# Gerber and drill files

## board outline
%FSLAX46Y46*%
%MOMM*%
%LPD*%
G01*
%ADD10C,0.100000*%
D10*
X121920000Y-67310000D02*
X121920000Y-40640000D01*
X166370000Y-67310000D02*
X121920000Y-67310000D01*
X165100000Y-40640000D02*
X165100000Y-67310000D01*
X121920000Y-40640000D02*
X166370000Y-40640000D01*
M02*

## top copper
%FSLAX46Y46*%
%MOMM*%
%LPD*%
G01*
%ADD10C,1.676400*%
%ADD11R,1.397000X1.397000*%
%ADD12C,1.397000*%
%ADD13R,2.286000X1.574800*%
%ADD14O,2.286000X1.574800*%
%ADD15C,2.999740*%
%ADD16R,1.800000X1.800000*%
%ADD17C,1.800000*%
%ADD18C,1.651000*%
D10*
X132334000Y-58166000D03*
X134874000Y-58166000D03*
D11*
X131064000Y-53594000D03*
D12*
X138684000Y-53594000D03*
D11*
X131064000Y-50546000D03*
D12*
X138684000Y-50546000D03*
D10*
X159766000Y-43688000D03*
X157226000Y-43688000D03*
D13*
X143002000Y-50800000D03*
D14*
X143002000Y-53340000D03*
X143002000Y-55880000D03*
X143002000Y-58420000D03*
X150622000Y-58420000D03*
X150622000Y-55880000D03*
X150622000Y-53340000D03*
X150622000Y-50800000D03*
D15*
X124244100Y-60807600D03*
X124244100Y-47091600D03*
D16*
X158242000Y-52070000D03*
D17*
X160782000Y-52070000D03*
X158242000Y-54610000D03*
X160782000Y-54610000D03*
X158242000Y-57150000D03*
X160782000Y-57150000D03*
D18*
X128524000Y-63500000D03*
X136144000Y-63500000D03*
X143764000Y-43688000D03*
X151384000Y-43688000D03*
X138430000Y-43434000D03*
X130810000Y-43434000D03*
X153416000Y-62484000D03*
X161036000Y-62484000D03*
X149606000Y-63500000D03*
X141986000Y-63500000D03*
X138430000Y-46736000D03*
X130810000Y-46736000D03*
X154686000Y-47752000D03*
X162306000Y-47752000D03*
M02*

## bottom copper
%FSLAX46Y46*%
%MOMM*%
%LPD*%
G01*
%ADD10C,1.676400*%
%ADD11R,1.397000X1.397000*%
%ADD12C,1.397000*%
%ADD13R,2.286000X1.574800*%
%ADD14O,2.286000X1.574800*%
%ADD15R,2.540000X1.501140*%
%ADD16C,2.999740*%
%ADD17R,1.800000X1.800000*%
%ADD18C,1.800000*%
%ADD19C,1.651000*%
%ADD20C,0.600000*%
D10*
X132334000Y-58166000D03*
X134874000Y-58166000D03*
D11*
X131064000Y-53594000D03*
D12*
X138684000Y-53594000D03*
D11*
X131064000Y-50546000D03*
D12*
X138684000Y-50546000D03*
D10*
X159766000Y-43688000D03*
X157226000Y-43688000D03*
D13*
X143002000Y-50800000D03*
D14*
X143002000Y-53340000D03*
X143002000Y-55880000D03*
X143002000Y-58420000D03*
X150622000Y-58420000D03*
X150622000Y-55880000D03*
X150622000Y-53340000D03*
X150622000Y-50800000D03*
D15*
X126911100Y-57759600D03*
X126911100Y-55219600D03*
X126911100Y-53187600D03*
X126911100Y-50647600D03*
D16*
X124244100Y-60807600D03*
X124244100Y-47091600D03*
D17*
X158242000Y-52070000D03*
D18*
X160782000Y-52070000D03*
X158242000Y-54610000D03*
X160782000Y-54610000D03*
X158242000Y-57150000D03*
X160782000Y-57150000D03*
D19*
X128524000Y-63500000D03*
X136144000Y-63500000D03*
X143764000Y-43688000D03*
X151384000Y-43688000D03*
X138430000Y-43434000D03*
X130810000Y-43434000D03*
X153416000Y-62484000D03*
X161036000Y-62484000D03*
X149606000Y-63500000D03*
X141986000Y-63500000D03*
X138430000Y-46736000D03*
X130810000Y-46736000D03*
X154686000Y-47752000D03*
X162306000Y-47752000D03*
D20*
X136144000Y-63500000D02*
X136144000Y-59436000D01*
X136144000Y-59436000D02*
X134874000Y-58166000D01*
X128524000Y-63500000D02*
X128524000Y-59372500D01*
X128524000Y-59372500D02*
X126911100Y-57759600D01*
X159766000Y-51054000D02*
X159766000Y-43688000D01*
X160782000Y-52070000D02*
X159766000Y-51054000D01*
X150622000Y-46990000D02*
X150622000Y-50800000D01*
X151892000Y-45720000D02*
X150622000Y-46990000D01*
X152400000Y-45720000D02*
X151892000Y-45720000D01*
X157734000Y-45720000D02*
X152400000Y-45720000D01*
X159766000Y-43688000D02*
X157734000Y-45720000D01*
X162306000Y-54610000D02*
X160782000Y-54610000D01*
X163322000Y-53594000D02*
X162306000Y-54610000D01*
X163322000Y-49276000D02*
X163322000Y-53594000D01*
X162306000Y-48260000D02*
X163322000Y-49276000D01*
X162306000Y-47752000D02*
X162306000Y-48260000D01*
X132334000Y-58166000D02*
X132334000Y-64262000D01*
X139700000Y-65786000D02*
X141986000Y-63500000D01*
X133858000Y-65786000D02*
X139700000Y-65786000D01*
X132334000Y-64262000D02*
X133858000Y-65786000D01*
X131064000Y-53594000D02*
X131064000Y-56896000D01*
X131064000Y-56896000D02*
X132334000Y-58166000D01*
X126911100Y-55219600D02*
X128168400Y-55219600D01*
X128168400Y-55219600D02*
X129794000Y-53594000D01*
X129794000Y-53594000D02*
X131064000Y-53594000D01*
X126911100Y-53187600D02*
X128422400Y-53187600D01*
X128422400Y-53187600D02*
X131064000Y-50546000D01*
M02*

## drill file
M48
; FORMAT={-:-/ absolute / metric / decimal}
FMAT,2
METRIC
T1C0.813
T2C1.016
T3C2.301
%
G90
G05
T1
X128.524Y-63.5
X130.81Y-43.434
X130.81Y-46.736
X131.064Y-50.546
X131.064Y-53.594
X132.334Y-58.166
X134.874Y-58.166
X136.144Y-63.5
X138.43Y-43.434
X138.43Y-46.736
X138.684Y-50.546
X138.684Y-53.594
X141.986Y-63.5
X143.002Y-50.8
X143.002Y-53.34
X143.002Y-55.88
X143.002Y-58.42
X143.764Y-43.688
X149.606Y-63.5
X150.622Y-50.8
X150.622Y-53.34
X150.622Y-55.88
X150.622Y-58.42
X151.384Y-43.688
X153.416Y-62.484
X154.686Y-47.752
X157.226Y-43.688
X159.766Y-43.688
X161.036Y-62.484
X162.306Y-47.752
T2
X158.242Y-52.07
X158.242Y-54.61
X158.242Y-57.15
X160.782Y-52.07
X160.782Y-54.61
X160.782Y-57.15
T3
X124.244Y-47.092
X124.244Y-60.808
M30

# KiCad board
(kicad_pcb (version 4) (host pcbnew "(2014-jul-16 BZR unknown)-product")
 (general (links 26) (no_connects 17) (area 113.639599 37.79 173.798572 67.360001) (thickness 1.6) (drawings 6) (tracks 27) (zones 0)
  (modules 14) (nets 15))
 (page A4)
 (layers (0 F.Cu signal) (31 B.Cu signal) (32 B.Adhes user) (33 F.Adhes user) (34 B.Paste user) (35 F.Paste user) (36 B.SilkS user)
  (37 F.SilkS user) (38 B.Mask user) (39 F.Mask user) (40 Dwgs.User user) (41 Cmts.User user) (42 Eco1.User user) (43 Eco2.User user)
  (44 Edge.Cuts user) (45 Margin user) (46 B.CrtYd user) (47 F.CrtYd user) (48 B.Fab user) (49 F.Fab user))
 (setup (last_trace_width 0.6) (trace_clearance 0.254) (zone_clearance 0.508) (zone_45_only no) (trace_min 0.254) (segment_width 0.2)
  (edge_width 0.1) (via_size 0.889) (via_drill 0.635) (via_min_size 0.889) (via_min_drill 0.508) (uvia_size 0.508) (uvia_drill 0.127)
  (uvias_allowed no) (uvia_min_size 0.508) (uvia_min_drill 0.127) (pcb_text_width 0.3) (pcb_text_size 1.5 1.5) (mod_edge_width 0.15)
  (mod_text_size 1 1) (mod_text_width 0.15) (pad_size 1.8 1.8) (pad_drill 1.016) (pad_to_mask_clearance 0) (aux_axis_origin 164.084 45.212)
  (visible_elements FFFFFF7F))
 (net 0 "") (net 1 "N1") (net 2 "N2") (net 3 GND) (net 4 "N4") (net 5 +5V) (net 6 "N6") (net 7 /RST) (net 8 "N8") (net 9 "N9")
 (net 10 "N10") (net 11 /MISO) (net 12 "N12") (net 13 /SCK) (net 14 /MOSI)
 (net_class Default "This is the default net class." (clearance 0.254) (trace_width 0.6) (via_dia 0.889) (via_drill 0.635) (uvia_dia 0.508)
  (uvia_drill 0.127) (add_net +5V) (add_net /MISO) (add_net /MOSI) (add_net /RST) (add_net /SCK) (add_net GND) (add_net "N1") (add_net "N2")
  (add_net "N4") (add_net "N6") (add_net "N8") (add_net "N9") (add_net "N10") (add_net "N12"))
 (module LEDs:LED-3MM (layer F.Cu) (at 133.604 58.166)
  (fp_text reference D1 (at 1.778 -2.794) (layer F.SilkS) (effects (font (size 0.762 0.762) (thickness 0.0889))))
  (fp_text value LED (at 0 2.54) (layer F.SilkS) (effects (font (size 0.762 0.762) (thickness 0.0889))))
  (pad 1 thru_hole circle (at -1.27 0) (size 1.6764 1.6764) (drill 0.8128) (layers *.Cu *.Mask F.SilkS) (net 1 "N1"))
  (pad 2 thru_hole circle (at 1.27 0) (size 1.6764 1.6764) (drill 0.8128) (layers *.Cu *.Mask F.SilkS) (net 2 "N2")))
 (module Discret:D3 (layer F.Cu) (at 134.874 53.594 180)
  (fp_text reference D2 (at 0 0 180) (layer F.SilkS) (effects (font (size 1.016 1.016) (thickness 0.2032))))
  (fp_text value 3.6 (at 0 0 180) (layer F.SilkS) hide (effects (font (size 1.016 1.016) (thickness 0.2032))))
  (pad 2 thru_hole rect (at 3.81 0 180) (size 1.397 1.397) (drill 0.8128) (layers *.Cu *.Mask F.SilkS) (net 1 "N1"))
  (pad 1 thru_hole circle (at -3.81 0 180) (size 1.397 1.397) (drill 0.8128) (layers *.Cu *.Mask F.SilkS) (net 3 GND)))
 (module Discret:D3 (layer F.Cu) (at 134.874 50.546 180)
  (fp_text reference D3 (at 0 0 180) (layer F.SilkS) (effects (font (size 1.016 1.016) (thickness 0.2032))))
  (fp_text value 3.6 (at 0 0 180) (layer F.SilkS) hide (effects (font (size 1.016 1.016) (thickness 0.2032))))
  (pad 2 thru_hole rect (at 3.81 0 180) (size 1.397 1.397) (drill 0.8128) (layers *.Cu *.Mask F.SilkS) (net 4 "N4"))
  (pad 1 thru_hole circle (at -3.81 0 180) (size 1.397 1.397) (drill 0.8128) (layers *.Cu *.Mask F.SilkS) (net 3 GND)))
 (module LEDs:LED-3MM (layer F.Cu) (at 158.496 43.688 180)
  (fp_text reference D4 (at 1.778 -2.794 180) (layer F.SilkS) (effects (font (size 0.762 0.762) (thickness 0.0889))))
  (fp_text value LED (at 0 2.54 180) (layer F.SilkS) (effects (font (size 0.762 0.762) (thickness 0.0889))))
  (pad 1 thru_hole circle (at -1.27 0 180) (size 1.6764 1.6764) (drill 0.8128) (layers *.Cu *.Mask F.SilkS) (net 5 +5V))
  (pad 2 thru_hole circle (at 1.27 0 180) (size 1.6764 1.6764) (drill 0.8128) (layers *.Cu *.Mask F.SilkS) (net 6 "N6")))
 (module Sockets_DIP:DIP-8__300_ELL (layer F.Cu) (at 146.812 54.61 270)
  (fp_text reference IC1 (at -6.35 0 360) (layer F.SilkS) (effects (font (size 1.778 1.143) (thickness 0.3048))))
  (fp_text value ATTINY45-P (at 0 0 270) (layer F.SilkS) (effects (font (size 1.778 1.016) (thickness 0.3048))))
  (pad 1 thru_hole rect (at -3.81 3.81 270) (size 1.5748 2.286) (drill 0.8128) (layers *.Cu *.Mask F.SilkS) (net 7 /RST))
  (pad 2 thru_hole oval (at -1.27 3.81 270) (size 1.5748 2.286) (drill 0.8128) (layers *.Cu *.Mask F.SilkS) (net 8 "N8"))
  (pad 3 thru_hole oval (at 1.27 3.81 270) (size 1.5748 2.286) (drill 0.8128) (layers *.Cu *.Mask F.SilkS) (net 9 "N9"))
  (pad 4 thru_hole oval (at 3.81 3.81 270) (size 1.5748 2.286) (drill 0.8128) (layers *.Cu *.Mask F.SilkS) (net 3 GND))
  (pad 5 thru_hole oval (at 3.81 -3.81 270) (size 1.5748 2.286) (drill 0.8128) (layers *.Cu *.Mask F.SilkS) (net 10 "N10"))
  (pad 6 thru_hole oval (at 1.27 -3.81 270) (size 1.5748 2.286) (drill 0.8128) (layers *.Cu *.Mask F.SilkS) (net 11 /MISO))
  (pad 7 thru_hole oval (at -1.27 -3.81 270) (size 1.5748 2.286) (drill 0.8128) (layers *.Cu *.Mask F.SilkS) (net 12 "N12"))
  (pad 8 thru_hole oval (at -3.81 -3.81 270) (size 1.5748 2.286) (drill 0.8128) (layers *.Cu *.Mask F.SilkS) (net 5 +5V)))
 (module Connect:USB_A (layer F.Cu) (at 126.9111 54.2036 180)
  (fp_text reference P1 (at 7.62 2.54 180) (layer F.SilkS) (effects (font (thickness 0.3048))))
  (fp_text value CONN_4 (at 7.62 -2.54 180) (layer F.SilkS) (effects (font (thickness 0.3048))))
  (pad 4 smd rect (at 0 -3.556 180) (size 2.54 1.50114) (layers B.Cu F.Paste F.Mask) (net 3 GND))
  (pad 3 smd rect (at 0 -1.016 180) (size 2.54 1.50114) (layers B.Cu F.Paste F.Mask) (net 1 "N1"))
  (pad 2 smd rect (at 0 1.016 180) (size 2.54 1.50114) (layers B.Cu F.Paste F.Mask) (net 4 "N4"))
  (pad 1 smd rect (at 0 3.556 180) (size 2.54 1.50114) (layers B.Cu F.Paste F.Mask) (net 5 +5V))
  (pad 5 thru_hole circle (at 2.667 -6.604 180) (size 2.99974 2.99974) (drill 2.30124) (layers *.Cu *.Mask F.SilkS))
  (pad 6 thru_hole circle (at 2.667 7.112 180) (size 2.99974 2.99974) (drill 2.30124) (layers *.Cu *.Mask F.SilkS)))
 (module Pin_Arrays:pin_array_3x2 (layer F.Cu) (at 159.512 54.61 270)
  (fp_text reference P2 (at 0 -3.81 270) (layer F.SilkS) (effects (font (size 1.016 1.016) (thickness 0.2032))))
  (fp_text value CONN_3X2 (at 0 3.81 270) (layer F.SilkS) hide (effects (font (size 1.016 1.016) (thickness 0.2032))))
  (pad 1 thru_hole rect (at -2.54 1.27 270) (size 1.8 1.8) (drill 1.016) (layers *.Cu *.Mask F.SilkS) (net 11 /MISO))
  (pad 2 thru_hole circle (at -2.54 -1.27 270) (size 1.8 1.8) (drill 1.016) (layers *.Cu *.Mask F.SilkS) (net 5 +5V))
  (pad 3 thru_hole circle (at 0 1.27 270) (size 1.8 1.8) (drill 1.016) (layers *.Cu *.Mask F.SilkS) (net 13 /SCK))
  (pad 4 thru_hole circle (at 0 -1.27 270) (size 1.8 1.8) (drill 1.016) (layers *.Cu *.Mask F.SilkS) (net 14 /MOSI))
  (pad e thru_hole circle (at 2.54 1.27 270) (size 1.8 1.8) (drill 1.016) (layers *.Cu *.Mask F.SilkS) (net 7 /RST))
  (pad 6 thru_hole circle (at 2.54 -1.27 270) (size 1.8 1.8) (drill 1.016) (layers *.Cu *.Mask F.SilkS) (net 3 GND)))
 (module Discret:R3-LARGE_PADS (layer F.Cu) (at 132.334 63.5) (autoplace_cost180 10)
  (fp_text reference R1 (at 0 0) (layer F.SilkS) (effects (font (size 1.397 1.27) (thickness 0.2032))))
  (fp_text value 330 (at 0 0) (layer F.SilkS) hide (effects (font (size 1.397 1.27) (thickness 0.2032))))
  (pad 1 thru_hole circle (at -3.81 0) (size 1.651 1.651) (drill 0.8128) (layers *.Cu *.Mask F.SilkS) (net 3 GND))
  (pad 2 thru_hole circle (at 3.81 0) (size 1.651 1.651) (drill 0.8128) (layers *.Cu *.Mask F.SilkS) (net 2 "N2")))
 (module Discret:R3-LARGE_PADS (layer F.Cu) (at 147.574 43.688) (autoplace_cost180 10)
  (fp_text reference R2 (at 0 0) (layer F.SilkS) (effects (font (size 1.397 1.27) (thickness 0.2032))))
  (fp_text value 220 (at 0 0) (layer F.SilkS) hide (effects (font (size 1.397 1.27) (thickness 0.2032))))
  (pad 1 thru_hole circle (at -3.81 0) (size 1.651 1.651) (drill 0.8128) (layers *.Cu *.Mask F.SilkS) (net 3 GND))
  (pad 2 thru_hole circle (at 3.81 0) (size 1.651 1.651) (drill 0.8128) (layers *.Cu *.Mask F.SilkS) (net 6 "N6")))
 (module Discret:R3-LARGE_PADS (layer F.Cu) (at 134.62 43.434 180) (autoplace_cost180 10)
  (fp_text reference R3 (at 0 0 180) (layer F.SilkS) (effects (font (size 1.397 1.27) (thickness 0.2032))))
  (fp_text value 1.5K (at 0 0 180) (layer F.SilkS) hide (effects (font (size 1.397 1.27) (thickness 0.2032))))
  (pad 1 thru_hole circle (at -3.81 0 180) (size 1.651 1.651) (drill 0.8128) (layers *.Cu *.Mask F.SilkS) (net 5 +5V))
  (pad 2 thru_hole circle (at 3.81 0 180) (size 1.651 1.651) (drill 0.8128) (layers *.Cu *.Mask F.SilkS) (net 4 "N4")))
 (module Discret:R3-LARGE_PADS (layer F.Cu) (at 157.226 62.484) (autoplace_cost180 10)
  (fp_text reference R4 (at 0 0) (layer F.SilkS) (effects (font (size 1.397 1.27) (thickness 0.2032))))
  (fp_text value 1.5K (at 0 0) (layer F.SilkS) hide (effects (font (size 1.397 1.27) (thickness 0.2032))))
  (pad 1 thru_hole circle (at -3.81 0) (size 1.651 1.651) (drill 0.8128) (layers *.Cu *.Mask F.SilkS) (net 12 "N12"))
  (pad 2 thru_hole circle (at 3.81 0) (size 1.651 1.651) (drill 0.8128) (layers *.Cu *.Mask F.SilkS) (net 13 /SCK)))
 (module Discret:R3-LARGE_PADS (layer F.Cu) (at 145.796 63.5 180) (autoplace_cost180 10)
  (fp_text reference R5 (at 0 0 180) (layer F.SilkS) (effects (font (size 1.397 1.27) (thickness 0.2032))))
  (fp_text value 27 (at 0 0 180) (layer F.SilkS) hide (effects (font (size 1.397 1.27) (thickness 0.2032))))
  (pad 1 thru_hole circle (at -3.81 0 180) (size 1.651 1.651) (drill 0.8128) (layers *.Cu *.Mask F.SilkS) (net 8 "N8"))
  (pad 2 thru_hole circle (at 3.81 0 180) (size 1.651 1.651) (drill 0.8128) (layers *.Cu *.Mask F.SilkS) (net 1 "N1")))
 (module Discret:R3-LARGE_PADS (layer F.Cu) (at 134.62 46.736 180) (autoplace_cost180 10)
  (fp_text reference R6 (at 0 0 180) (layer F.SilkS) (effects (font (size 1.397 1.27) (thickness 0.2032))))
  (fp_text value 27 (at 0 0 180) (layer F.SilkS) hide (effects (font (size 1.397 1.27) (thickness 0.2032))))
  (pad 1 thru_hole circle (at -3.81 0 180) (size 1.651 1.651) (drill 0.8128) (layers *.Cu *.Mask F.SilkS) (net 9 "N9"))
  (pad 2 thru_hole circle (at 3.81 0 180) (size 1.651 1.651) (drill 0.8128) (layers *.Cu *.Mask F.SilkS) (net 4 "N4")))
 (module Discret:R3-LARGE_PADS (layer F.Cu) (at 158.496 47.752) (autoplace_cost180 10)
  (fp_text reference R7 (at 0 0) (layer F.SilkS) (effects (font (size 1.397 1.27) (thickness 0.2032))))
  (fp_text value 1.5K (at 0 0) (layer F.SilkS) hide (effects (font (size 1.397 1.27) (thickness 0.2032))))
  (pad 1 thru_hole circle (at -3.81 0) (size 1.651 1.651) (drill 0.8128) (layers *.Cu *.Mask F.SilkS) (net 10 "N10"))
  (pad 2 thru_hole circle (at 3.81 0) (size 1.651 1.651) (drill 0.8128) (layers *.Cu *.Mask F.SilkS) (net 14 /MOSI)))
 (gr_line (start 121.92 67.31) (end 121.92 40.64) (angle 90) (layer Edge.Cuts) (width 0.1))
 (gr_line (start 166.37 67.31) (end 121.92 67.31) (angle 90) (layer Edge.Cuts) (width 0.1))
 (gr_line (start 165.1 40.64) (end 165.1 67.31) (angle 90) (layer Edge.Cuts) (width 0.1))
 (gr_line (start 121.92 40.64) (end 166.37 40.64) (angle 90) (layer Edge.Cuts) (width 0.1))
 (segment (start 136.144 63.5) (end 136.144 59.436) (width 0.6) (layer B.Cu) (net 2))
 (segment (start 136.144 59.436) (end 134.874 58.166) (width 0.6) (layer B.Cu) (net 2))
 (segment (start 128.524 63.5) (end 128.524 59.3725) (width 0.6) (layer B.Cu) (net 3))
 (segment (start 128.524 59.3725) (end 126.9111 57.7596) (width 0.6) (layer B.Cu) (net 3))
 (segment (start 159.766 51.054) (end 159.766 43.688) (width 0.6) (layer B.Cu) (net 5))
 (segment (start 160.782 52.07) (end 159.766 51.054) (width 0.6) (layer B.Cu) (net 5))
 (segment (start 150.622 46.99) (end 150.622 50.8) (width 0.6) (layer B.Cu) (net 5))
 (segment (start 151.892 45.72) (end 150.622 46.99) (width 0.6) (layer B.Cu) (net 5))
 (segment (start 152.4 45.72) (end 151.892 45.72) (width 0.6) (layer B.Cu) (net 5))
 (segment (start 157.734 45.72) (end 152.4 45.72) (width 0.6) (layer B.Cu) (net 5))
 (segment (start 159.766 43.688) (end 157.734 45.72) (width 0.6) (layer B.Cu) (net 5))
 (segment (start 162.306 54.61) (end 160.782 54.61) (width 0.6) (layer B.Cu) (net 14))
 (segment (start 163.322 53.594) (end 162.306 54.61) (width 0.6) (layer B.Cu) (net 14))
 (segment (start 163.322 49.276) (end 163.322 53.594) (width 0.6) (layer B.Cu) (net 14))
 (segment (start 162.306 48.26) (end 163.322 49.276) (width 0.6) (layer B.Cu) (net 14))
 (segment (start 162.306 47.752) (end 162.306 48.26) (width 0.6) (layer B.Cu) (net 14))
 (segment (start 132.334 58.166) (end 132.334 64.262) (width 0.6) (layer B.Cu) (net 1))
 (segment (start 139.7 65.786) (end 141.986 63.5) (width 0.6) (layer B.Cu) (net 1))
 (segment (start 133.858 65.786) (end 139.7 65.786) (width 0.6) (layer B.Cu) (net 1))
 (segment (start 132.334 64.262) (end 133.858 65.786) (width 0.6) (layer B.Cu) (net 1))
 (segment (start 131.064 53.594) (end 131.064 56.896) (width 0.6) (layer B.Cu) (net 1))
 (segment (start 131.064 56.896) (end 132.334 58.166) (width 0.6) (layer B.Cu) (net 1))
 (segment (start 126.9111 55.2196) (end 128.1684 55.2196) (width 0.6) (layer B.Cu) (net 1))
 (segment (start 128.1684 55.2196) (end 129.794 53.594) (width 0.6) (layer B.Cu) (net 1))
 (segment (start 129.794 53.594) (end 131.064 53.594) (width 0.6) (layer B.Cu) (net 1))
 (segment (start 126.9111 53.1876) (end 128.4224 53.1876) (width 0.6) (layer B.Cu) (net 4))
 (segment (start 128.4224 53.1876) (end 131.064 50.546) (width 0.6) (layer B.Cu) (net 4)))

